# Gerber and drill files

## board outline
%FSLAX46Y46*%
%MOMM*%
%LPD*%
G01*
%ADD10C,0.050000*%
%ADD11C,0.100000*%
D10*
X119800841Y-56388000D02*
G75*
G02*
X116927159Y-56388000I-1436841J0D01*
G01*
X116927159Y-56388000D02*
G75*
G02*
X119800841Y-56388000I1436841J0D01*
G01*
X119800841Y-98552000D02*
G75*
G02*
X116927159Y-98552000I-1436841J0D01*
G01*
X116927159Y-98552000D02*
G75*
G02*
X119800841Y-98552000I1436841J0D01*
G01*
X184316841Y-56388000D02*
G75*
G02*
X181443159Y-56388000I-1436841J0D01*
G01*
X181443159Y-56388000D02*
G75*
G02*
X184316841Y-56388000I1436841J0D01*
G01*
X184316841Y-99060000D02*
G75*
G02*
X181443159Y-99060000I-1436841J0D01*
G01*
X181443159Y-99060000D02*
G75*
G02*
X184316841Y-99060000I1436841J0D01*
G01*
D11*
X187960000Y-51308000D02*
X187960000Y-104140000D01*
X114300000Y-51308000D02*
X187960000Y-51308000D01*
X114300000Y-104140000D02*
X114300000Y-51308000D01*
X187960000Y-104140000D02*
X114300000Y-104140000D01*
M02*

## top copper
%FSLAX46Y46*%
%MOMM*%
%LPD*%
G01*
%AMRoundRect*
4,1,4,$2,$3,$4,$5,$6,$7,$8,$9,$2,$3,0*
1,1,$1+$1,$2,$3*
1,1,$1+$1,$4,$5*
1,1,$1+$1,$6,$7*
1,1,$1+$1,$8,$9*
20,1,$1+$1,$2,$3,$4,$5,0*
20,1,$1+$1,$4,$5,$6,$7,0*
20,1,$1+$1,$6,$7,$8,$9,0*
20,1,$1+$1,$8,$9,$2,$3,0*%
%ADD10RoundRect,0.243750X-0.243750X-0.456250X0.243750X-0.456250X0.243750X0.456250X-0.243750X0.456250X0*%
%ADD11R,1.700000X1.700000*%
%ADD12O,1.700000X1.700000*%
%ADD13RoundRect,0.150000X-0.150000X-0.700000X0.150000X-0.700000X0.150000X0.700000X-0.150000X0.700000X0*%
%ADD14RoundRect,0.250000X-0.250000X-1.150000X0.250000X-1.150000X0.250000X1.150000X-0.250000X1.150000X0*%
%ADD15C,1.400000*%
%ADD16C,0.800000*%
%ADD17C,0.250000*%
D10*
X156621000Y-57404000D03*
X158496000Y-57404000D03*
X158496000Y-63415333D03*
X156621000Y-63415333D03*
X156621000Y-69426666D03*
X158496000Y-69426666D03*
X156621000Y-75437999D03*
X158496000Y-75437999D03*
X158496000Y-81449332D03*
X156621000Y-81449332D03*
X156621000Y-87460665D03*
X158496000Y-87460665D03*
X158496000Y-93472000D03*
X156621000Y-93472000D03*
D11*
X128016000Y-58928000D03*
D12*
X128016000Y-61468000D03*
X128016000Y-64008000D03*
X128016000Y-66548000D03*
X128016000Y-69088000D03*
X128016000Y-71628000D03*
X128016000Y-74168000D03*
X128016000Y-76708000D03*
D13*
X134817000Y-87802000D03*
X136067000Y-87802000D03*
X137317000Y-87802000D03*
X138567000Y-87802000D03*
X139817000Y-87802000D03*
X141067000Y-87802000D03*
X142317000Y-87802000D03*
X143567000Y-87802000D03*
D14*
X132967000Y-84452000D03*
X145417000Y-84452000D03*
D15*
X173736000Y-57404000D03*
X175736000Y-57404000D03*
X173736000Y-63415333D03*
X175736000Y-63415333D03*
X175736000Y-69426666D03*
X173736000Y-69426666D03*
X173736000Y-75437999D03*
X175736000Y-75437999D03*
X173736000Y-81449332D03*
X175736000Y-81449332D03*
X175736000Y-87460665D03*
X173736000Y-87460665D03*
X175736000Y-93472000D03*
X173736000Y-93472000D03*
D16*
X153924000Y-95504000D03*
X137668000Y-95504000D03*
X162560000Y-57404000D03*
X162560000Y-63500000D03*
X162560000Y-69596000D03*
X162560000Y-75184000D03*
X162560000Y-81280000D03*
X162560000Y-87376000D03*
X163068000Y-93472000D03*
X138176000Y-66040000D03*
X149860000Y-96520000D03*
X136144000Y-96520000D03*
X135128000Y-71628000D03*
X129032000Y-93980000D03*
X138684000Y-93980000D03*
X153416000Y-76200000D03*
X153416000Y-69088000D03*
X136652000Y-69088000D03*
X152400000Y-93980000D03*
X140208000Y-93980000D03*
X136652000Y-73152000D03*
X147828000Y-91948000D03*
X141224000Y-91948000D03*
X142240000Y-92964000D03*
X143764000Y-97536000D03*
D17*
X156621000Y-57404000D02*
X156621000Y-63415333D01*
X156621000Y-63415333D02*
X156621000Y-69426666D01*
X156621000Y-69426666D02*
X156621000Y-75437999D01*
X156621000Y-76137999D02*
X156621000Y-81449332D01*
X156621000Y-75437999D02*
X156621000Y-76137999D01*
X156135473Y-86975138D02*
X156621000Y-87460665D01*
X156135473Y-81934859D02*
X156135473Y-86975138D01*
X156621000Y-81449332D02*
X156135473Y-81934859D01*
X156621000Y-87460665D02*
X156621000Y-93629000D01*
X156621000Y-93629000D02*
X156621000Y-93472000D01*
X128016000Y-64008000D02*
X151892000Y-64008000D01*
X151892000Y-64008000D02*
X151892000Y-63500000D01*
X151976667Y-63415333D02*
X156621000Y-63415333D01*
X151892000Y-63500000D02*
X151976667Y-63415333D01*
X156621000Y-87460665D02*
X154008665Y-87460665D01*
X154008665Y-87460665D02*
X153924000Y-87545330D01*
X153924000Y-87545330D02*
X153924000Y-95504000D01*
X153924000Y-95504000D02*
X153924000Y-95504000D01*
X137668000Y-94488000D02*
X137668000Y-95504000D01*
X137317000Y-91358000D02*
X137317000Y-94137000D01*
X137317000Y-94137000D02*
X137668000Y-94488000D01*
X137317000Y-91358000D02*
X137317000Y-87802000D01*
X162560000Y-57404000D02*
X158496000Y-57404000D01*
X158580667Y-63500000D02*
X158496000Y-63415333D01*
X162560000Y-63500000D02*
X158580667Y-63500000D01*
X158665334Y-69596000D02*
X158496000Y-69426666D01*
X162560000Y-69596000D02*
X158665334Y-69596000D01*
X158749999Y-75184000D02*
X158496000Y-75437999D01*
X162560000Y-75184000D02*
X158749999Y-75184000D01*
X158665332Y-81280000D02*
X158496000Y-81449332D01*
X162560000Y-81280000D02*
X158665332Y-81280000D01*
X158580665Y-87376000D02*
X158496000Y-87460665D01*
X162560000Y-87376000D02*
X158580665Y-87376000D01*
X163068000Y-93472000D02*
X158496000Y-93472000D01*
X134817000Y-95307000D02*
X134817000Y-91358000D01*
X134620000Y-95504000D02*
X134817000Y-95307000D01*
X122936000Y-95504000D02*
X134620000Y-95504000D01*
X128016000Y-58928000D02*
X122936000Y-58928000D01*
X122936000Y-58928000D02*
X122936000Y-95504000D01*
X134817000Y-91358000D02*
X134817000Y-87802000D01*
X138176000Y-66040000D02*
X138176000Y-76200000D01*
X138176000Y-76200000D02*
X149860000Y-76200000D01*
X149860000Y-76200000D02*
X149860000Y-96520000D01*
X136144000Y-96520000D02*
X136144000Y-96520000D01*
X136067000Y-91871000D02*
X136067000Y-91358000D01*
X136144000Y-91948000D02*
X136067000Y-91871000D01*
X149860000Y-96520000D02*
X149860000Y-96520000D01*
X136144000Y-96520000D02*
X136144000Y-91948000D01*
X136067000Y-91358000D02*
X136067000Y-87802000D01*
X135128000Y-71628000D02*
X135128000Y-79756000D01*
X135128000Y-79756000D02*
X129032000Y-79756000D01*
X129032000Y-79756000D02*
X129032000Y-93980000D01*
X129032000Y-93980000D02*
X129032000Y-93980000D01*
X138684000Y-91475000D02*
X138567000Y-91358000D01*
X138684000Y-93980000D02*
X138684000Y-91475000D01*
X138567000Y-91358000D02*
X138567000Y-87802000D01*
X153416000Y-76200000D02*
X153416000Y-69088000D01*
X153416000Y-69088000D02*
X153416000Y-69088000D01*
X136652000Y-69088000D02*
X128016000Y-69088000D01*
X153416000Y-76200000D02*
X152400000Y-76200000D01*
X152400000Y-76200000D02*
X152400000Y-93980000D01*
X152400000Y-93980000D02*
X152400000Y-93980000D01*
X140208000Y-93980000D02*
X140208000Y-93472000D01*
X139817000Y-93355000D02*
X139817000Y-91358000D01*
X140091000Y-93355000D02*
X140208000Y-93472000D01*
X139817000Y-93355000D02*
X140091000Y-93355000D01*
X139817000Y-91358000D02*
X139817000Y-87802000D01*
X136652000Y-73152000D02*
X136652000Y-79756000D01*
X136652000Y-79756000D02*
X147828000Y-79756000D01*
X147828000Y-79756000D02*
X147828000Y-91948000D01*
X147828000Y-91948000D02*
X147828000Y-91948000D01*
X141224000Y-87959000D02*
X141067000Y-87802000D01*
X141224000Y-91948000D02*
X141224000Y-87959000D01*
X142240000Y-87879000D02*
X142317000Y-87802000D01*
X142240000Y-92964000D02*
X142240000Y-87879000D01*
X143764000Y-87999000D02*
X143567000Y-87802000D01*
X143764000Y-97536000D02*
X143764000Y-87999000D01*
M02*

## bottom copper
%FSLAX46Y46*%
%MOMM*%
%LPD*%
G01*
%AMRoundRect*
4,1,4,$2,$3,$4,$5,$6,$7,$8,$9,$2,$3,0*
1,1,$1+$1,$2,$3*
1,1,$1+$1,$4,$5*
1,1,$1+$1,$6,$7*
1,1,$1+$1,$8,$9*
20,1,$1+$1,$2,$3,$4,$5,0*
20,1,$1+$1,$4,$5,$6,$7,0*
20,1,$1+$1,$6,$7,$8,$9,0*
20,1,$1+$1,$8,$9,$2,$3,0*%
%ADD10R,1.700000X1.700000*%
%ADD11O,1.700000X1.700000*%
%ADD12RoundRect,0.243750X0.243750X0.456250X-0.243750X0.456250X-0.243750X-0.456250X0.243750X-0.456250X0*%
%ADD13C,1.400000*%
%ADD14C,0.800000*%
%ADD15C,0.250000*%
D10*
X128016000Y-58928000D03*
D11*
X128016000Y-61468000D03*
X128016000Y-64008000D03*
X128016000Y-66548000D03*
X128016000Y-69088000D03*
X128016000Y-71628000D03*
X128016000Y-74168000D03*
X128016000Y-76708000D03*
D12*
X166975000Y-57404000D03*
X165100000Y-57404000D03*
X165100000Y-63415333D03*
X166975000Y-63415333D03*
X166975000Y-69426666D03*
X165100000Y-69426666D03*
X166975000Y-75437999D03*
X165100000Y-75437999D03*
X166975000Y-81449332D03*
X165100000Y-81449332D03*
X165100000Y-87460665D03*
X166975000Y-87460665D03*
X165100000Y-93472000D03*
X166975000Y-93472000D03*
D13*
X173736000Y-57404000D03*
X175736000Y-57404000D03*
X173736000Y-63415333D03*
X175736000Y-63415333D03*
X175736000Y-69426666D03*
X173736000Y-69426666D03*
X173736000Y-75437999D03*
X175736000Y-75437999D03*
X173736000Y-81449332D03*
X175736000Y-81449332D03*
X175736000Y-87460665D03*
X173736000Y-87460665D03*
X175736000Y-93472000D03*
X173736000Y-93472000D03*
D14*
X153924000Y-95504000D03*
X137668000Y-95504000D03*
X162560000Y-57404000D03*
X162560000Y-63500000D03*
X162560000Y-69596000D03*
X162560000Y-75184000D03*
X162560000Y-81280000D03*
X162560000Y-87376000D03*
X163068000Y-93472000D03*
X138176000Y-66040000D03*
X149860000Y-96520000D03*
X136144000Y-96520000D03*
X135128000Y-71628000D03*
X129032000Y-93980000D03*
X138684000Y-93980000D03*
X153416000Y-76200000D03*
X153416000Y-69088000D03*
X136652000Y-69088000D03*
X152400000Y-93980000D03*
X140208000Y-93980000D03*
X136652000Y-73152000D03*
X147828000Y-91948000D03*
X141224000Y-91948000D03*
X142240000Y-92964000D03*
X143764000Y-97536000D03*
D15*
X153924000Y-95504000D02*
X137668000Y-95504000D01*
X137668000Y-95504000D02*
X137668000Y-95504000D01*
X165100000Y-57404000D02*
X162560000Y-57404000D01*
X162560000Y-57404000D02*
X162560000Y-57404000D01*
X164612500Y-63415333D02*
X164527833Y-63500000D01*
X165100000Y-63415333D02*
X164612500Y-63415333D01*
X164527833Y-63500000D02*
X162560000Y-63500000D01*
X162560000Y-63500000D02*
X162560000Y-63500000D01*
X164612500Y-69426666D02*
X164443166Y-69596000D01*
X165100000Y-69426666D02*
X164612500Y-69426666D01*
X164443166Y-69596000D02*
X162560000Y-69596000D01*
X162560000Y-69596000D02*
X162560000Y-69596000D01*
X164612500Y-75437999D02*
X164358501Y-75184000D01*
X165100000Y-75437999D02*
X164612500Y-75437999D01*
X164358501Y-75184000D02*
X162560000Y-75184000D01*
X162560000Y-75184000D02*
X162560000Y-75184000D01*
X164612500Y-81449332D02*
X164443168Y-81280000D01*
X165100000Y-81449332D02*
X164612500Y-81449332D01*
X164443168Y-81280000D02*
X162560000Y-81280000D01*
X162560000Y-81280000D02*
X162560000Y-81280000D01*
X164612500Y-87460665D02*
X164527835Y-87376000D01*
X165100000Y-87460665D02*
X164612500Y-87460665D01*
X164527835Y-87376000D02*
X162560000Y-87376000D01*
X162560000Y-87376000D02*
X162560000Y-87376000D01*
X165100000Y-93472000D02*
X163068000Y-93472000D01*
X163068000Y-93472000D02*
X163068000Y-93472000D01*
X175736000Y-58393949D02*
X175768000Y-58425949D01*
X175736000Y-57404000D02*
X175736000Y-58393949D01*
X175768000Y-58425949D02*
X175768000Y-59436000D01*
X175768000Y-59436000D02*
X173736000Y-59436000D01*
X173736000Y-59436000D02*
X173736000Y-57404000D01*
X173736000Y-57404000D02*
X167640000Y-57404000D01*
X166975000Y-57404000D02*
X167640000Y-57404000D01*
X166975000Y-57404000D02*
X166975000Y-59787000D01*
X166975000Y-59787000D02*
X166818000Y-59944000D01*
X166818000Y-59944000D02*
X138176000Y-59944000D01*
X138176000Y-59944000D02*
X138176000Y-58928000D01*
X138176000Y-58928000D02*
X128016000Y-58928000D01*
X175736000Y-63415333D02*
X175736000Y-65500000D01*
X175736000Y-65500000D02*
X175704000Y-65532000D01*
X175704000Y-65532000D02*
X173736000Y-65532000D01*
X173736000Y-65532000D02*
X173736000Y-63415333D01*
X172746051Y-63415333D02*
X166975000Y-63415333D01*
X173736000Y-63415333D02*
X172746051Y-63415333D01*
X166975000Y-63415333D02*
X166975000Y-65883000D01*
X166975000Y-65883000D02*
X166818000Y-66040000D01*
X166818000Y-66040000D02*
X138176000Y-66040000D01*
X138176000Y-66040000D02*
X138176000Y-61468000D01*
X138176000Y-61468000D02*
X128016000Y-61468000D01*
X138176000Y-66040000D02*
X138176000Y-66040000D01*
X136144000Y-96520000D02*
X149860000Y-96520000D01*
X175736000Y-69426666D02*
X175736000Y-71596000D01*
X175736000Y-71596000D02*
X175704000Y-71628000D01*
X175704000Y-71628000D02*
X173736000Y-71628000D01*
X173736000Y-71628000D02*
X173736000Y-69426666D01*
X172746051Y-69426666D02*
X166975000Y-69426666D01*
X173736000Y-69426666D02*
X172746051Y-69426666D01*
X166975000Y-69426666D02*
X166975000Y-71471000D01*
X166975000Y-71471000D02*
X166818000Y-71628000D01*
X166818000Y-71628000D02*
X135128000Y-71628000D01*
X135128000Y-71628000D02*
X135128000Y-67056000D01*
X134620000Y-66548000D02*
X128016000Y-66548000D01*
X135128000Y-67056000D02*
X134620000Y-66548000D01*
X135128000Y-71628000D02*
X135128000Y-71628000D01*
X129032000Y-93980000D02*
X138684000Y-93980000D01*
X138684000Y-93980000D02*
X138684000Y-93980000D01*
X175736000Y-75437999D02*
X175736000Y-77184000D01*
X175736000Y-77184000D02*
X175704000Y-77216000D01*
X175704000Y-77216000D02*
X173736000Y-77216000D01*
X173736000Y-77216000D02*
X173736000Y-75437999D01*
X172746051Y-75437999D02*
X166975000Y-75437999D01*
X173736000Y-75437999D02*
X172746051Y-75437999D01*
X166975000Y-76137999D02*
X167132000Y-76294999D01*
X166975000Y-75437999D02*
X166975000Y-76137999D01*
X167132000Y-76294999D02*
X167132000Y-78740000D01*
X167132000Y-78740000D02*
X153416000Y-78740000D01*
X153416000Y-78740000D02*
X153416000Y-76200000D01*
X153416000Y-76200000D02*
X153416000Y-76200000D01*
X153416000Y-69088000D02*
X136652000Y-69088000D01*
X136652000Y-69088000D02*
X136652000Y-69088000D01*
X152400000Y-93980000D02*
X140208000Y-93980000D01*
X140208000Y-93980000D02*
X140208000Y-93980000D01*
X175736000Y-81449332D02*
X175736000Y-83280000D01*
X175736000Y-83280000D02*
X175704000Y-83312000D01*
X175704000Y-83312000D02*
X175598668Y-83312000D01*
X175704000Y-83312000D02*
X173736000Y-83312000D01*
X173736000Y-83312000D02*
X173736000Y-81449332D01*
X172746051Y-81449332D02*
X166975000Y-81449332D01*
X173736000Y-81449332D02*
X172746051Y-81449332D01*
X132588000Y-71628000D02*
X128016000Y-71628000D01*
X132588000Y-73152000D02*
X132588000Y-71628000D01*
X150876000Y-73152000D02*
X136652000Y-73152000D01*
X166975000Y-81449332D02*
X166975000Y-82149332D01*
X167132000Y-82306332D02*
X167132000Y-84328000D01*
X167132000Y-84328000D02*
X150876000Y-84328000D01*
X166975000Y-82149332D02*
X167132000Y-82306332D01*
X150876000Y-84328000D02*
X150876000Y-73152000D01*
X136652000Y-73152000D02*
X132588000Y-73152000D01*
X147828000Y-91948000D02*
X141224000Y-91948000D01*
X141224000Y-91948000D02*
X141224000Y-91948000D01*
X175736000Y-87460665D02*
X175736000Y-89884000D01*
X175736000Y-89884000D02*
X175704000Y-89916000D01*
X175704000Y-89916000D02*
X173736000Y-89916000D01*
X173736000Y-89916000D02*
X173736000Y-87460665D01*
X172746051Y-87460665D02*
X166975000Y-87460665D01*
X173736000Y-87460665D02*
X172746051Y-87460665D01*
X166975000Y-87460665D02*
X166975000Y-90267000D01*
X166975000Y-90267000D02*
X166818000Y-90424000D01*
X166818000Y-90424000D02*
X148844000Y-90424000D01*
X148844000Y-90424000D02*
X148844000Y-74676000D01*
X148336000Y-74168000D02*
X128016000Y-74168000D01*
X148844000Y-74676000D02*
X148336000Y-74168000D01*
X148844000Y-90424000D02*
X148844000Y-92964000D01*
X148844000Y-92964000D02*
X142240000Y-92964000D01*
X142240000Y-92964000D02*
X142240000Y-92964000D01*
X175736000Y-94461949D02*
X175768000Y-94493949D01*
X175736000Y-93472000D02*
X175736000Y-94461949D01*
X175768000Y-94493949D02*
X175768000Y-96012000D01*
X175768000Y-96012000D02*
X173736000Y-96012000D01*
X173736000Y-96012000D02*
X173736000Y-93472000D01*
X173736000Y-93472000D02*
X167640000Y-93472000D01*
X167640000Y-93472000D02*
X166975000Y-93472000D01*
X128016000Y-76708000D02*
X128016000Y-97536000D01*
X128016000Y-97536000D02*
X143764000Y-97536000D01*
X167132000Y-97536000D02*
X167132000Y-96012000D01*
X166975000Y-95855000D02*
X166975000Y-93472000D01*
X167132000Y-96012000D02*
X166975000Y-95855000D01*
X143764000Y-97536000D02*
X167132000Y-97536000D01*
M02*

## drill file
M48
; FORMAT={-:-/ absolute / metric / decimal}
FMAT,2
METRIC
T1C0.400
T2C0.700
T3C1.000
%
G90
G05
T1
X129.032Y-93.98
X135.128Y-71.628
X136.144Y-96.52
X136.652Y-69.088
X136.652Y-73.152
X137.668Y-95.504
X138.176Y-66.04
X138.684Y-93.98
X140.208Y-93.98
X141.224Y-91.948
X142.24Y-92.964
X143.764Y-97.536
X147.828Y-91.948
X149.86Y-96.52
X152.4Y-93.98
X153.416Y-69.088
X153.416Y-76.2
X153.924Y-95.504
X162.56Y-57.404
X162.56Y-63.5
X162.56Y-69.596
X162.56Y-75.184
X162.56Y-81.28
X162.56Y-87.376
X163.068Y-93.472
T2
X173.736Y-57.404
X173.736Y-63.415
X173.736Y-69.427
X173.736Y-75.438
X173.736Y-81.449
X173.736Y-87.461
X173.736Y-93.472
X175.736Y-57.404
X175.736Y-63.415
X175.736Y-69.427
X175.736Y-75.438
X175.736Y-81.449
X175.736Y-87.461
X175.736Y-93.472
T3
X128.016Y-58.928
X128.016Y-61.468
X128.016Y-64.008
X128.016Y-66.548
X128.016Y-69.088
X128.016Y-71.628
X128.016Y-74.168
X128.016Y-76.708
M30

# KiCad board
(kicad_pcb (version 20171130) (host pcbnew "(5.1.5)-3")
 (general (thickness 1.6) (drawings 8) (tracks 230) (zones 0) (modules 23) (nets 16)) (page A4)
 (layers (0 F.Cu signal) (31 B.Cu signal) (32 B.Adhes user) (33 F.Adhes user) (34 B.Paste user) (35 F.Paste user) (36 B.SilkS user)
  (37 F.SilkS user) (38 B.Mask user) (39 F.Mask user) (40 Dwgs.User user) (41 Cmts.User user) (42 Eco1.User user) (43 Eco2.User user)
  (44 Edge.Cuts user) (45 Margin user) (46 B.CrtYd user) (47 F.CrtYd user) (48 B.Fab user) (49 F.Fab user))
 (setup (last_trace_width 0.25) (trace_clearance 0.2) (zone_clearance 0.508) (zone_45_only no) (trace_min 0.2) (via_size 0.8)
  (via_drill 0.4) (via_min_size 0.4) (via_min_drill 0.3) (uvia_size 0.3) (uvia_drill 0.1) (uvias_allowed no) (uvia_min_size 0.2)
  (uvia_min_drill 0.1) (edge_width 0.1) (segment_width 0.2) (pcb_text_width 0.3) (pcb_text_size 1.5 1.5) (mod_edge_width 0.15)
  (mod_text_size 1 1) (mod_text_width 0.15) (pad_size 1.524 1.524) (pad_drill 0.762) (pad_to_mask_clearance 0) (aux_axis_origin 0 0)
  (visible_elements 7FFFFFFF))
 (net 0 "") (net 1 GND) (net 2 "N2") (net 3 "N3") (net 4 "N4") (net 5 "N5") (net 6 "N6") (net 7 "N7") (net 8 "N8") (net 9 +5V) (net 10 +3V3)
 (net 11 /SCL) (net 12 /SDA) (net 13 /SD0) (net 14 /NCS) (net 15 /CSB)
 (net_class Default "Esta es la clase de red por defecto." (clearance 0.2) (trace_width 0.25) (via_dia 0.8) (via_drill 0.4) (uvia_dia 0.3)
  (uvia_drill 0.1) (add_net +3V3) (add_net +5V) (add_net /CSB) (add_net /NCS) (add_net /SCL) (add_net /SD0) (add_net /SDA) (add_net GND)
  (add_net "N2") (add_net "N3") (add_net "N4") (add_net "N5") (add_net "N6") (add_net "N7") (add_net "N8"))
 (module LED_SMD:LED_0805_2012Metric (layer F.Cu) (at 157.5585 57.404)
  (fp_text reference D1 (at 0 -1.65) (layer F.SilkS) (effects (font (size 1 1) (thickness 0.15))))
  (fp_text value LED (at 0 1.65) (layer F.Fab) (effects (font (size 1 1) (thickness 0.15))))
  (pad 1 smd roundrect (at -0.9375 0) (size 0.975 1.4) (layers F.Cu F.Paste F.Mask) (roundrect_rratio 0.25) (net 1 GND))
  (pad 2 smd roundrect (at 0.9375 0) (size 0.975 1.4) (layers F.Cu F.Paste F.Mask) (roundrect_rratio 0.25) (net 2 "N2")))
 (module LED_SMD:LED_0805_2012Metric (layer F.Cu) (at 157.5585 63.415333)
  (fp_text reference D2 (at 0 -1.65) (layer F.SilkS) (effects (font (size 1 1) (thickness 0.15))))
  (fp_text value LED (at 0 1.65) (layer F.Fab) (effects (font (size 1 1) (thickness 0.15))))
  (pad 2 smd roundrect (at 0.9375 0) (size 0.975 1.4) (layers F.Cu F.Paste F.Mask) (roundrect_rratio 0.25) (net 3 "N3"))
  (pad 1 smd roundrect (at -0.9375 0) (size 0.975 1.4) (layers F.Cu F.Paste F.Mask) (roundrect_rratio 0.25) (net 1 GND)))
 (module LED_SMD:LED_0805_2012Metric (layer F.Cu) (at 157.5585 69.426666)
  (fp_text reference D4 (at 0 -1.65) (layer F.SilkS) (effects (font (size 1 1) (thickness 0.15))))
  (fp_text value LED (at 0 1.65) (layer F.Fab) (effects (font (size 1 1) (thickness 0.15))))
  (pad 1 smd roundrect (at -0.9375 0) (size 0.975 1.4) (layers F.Cu F.Paste F.Mask) (roundrect_rratio 0.25) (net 1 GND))
  (pad 2 smd roundrect (at 0.9375 0) (size 0.975 1.4) (layers F.Cu F.Paste F.Mask) (roundrect_rratio 0.25) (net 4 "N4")))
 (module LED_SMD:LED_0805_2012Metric (layer F.Cu) (at 157.5585 75.437999)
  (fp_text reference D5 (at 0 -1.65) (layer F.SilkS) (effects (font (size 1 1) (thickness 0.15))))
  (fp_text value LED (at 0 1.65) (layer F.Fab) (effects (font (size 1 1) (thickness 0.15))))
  (pad 1 smd roundrect (at -0.9375 0) (size 0.975 1.4) (layers F.Cu F.Paste F.Mask) (roundrect_rratio 0.25) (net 1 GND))
  (pad 2 smd roundrect (at 0.9375 0) (size 0.975 1.4) (layers F.Cu F.Paste F.Mask) (roundrect_rratio 0.25) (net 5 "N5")))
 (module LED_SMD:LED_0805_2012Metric (layer F.Cu) (at 157.5585 81.449332)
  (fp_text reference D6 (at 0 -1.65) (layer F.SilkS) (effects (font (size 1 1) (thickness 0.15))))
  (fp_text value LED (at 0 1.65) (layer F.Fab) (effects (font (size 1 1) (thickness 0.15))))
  (pad 2 smd roundrect (at 0.9375 0) (size 0.975 1.4) (layers F.Cu F.Paste F.Mask) (roundrect_rratio 0.25) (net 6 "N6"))
  (pad 1 smd roundrect (at -0.9375 0) (size 0.975 1.4) (layers F.Cu F.Paste F.Mask) (roundrect_rratio 0.25) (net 1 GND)))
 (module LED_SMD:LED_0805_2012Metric (layer F.Cu) (at 157.5585 87.460665)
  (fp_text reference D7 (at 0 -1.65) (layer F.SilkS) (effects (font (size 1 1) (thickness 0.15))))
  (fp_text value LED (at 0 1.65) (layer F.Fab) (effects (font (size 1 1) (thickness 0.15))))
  (pad 1 smd roundrect (at -0.9375 0) (size 0.975 1.4) (layers F.Cu F.Paste F.Mask) (roundrect_rratio 0.25) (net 1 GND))
  (pad 2 smd roundrect (at 0.9375 0) (size 0.975 1.4) (layers F.Cu F.Paste F.Mask) (roundrect_rratio 0.25) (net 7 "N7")))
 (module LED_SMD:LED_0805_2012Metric (layer F.Cu) (at 157.5585 93.472)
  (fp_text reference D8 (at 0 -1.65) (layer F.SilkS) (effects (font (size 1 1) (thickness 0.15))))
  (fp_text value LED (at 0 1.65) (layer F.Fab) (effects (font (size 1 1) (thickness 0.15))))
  (pad 2 smd roundrect (at 0.9375 0) (size 0.975 1.4) (layers F.Cu F.Paste F.Mask) (roundrect_rratio 0.25) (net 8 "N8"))
  (pad 1 smd roundrect (at -0.9375 0) (size 0.975 1.4) (layers F.Cu F.Paste F.Mask) (roundrect_rratio 0.25) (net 1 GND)))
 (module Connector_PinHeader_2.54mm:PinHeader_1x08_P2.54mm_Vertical (layer F.Cu) (at 128.016 58.928)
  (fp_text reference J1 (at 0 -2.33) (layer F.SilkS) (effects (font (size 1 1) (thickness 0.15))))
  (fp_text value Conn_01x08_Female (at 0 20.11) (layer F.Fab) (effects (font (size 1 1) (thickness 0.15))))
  (pad 1 thru_hole rect (at 0 0) (size 1.7 1.7) (drill 1) (layers *.Cu *.Mask) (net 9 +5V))
  (pad 2 thru_hole oval (at 0 2.54) (size 1.7 1.7) (drill 1) (layers *.Cu *.Mask) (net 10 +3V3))
  (pad 3 thru_hole oval (at 0 5.08) (size 1.7 1.7) (drill 1) (layers *.Cu *.Mask) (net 1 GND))
  (pad 4 thru_hole oval (at 0 7.62) (size 1.7 1.7) (drill 1) (layers *.Cu *.Mask) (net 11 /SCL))
  (pad 5 thru_hole oval (at 0 10.16) (size 1.7 1.7) (drill 1) (layers *.Cu *.Mask) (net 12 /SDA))
  (pad 6 thru_hole oval (at 0 12.7) (size 1.7 1.7) (drill 1) (layers *.Cu *.Mask) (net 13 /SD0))
  (pad 7 thru_hole oval (at 0 15.24) (size 1.7 1.7) (drill 1) (layers *.Cu *.Mask) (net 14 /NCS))
  (pad 8 thru_hole oval (at 0 17.78) (size 1.7 1.7) (drill 1) (layers *.Cu *.Mask) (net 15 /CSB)))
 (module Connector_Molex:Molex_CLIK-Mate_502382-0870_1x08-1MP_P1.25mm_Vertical (layer F.Cu) (at 139.192 85.852)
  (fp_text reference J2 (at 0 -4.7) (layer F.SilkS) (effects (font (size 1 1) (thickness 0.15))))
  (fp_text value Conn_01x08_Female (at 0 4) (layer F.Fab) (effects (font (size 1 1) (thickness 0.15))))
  (pad 1 smd roundrect (at -4.375 1.95) (size 0.6 1.7) (layers F.Cu F.Paste F.Mask) (roundrect_rratio 0.25) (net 9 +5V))
  (pad 2 smd roundrect (at -3.125 1.95) (size 0.6 1.7) (layers F.Cu F.Paste F.Mask) (roundrect_rratio 0.25) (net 10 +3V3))
  (pad 3 smd roundrect (at -1.875 1.95) (size 0.6 1.7) (layers F.Cu F.Paste F.Mask) (roundrect_rratio 0.25) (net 1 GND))
  (pad 4 smd roundrect (at -0.625 1.95) (size 0.6 1.7) (layers F.Cu F.Paste F.Mask) (roundrect_rratio 0.25) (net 11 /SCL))
  (pad 5 smd roundrect (at 0.625 1.95) (size 0.6 1.7) (layers F.Cu F.Paste F.Mask) (roundrect_rratio 0.25) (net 12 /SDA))
  (pad 6 smd roundrect (at 1.875 1.95) (size 0.6 1.7) (layers F.Cu F.Paste F.Mask) (roundrect_rratio 0.25) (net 13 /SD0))
  (pad 7 smd roundrect (at 3.125 1.95) (size 0.6 1.7) (layers F.Cu F.Paste F.Mask) (roundrect_rratio 0.25) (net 14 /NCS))
  (pad 8 smd roundrect (at 4.375 1.95) (size 0.6 1.7) (layers F.Cu F.Paste F.Mask) (roundrect_rratio 0.25) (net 15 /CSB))
  (pad MP smd roundrect (at -6.225 -1.4) (size 1 2.8) (layers F.Cu F.Paste F.Mask) (roundrect_rratio 0.25))
  (pad MP smd roundrect (at 6.225 -1.4) (size 1 2.8) (layers F.Cu F.Paste F.Mask) (roundrect_rratio 0.25)))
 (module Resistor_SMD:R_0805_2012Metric (layer B.Cu) (at 166.0375 57.404 180)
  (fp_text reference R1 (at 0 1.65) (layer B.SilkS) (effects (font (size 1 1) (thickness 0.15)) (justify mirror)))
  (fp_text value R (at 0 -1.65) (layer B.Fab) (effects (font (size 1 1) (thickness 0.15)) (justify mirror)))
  (pad 1 smd roundrect (at -0.9375 0 180) (size 0.975 1.4) (layers B.Cu B.Paste B.Mask) (roundrect_rratio 0.25) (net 9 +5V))
  (pad 2 smd roundrect (at 0.9375 0 180) (size 0.975 1.4) (layers B.Cu B.Paste B.Mask) (roundrect_rratio 0.25) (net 2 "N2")))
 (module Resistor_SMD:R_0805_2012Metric (layer B.Cu) (at 166.0375 63.415333 180)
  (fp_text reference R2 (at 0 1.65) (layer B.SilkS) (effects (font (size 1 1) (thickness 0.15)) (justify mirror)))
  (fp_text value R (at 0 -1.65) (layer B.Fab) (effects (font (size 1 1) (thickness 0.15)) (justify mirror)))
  (pad 2 smd roundrect (at 0.9375 0 180) (size 0.975 1.4) (layers B.Cu B.Paste B.Mask) (roundrect_rratio 0.25) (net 3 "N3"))
  (pad 1 smd roundrect (at -0.9375 0 180) (size 0.975 1.4) (layers B.Cu B.Paste B.Mask) (roundrect_rratio 0.25) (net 10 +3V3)))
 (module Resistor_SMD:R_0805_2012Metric (layer B.Cu) (at 166.0375 69.426666 180)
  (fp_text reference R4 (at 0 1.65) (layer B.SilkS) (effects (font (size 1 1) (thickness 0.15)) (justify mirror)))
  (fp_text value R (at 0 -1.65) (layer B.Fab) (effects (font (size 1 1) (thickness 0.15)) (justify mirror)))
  (pad 1 smd roundrect (at -0.9375 0 180) (size 0.975 1.4) (layers B.Cu B.Paste B.Mask) (roundrect_rratio 0.25) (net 11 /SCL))
  (pad 2 smd roundrect (at 0.9375 0 180) (size 0.975 1.4) (layers B.Cu B.Paste B.Mask) (roundrect_rratio 0.25) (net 4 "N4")))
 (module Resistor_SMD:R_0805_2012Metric (layer B.Cu) (at 166.0375 75.437999 180)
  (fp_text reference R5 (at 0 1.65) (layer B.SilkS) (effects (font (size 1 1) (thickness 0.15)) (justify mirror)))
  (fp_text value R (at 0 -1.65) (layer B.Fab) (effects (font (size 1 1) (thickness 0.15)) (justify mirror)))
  (pad 1 smd roundrect (at -0.9375 0 180) (size 0.975 1.4) (layers B.Cu B.Paste B.Mask) (roundrect_rratio 0.25) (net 12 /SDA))
  (pad 2 smd roundrect (at 0.9375 0 180) (size 0.975 1.4) (layers B.Cu B.Paste B.Mask) (roundrect_rratio 0.25) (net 5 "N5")))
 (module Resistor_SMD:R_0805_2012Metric (layer B.Cu) (at 166.0375 81.449332 180)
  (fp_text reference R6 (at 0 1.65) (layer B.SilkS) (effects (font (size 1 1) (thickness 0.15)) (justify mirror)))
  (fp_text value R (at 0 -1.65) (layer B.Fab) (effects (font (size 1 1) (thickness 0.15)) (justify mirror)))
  (pad 1 smd roundrect (at -0.9375 0 180) (size 0.975 1.4) (layers B.Cu B.Paste B.Mask) (roundrect_rratio 0.25) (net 13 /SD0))
  (pad 2 smd roundrect (at 0.9375 0 180) (size 0.975 1.4) (layers B.Cu B.Paste B.Mask) (roundrect_rratio 0.25) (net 6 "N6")))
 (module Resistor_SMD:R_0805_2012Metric (layer B.Cu) (at 166.0375 87.460665 180)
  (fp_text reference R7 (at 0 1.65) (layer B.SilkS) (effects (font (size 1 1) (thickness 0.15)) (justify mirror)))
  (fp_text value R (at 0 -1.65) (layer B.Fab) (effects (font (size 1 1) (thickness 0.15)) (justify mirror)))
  (pad 2 smd roundrect (at 0.9375 0 180) (size 0.975 1.4) (layers B.Cu B.Paste B.Mask) (roundrect_rratio 0.25) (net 7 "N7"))
  (pad 1 smd roundrect (at -0.9375 0 180) (size 0.975 1.4) (layers B.Cu B.Paste B.Mask) (roundrect_rratio 0.25) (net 14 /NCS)))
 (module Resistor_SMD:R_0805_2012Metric (layer B.Cu) (at 166.0375 93.472 180)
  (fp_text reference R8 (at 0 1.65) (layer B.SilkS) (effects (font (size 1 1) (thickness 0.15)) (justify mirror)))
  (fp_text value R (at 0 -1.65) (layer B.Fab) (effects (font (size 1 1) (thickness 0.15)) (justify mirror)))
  (pad 2 smd roundrect (at 0.9375 0 180) (size 0.975 1.4) (layers B.Cu B.Paste B.Mask) (roundrect_rratio 0.25) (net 8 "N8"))
  (pad 1 smd roundrect (at -0.9375 0 180) (size 0.975 1.4) (layers B.Cu B.Paste B.Mask) (roundrect_rratio 0.25) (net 15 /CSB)))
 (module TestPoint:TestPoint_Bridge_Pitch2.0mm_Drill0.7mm (layer F.Cu) (at 173.736 57.404)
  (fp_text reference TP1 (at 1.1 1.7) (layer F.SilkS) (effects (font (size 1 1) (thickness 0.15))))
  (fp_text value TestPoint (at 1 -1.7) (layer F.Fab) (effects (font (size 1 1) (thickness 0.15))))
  (pad 1 thru_hole circle (at 0 0) (size 1.4 1.4) (drill 0.7) (layers *.Cu *.Mask) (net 9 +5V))
  (pad 1 thru_hole circle (at 2 0) (size 1.4 1.4) (drill 0.7) (layers *.Cu *.Mask) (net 9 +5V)))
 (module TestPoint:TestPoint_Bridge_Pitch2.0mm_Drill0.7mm (layer F.Cu) (at 173.736 63.415333)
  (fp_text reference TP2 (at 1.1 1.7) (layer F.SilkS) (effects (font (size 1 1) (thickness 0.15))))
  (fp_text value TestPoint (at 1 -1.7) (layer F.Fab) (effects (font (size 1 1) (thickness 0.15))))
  (pad 1 thru_hole circle (at 0 0) (size 1.4 1.4) (drill 0.7) (layers *.Cu *.Mask) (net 10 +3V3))
  (pad 1 thru_hole circle (at 2 0) (size 1.4 1.4) (drill 0.7) (layers *.Cu *.Mask) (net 10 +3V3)))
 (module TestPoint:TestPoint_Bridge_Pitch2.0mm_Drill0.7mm (layer F.Cu) (at 173.736 69.426666)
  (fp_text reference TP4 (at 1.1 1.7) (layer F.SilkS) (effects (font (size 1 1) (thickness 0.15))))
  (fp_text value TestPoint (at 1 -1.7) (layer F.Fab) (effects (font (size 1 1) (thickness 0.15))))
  (pad 1 thru_hole circle (at 2 0) (size 1.4 1.4) (drill 0.7) (layers *.Cu *.Mask) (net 11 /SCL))
  (pad 1 thru_hole circle (at 0 0) (size 1.4 1.4) (drill 0.7) (layers *.Cu *.Mask) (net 11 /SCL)))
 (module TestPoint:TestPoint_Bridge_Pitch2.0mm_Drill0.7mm (layer F.Cu) (at 173.736 75.437999)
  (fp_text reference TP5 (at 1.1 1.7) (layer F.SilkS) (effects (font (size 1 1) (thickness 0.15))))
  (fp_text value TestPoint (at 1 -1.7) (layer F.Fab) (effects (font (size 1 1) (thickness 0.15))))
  (pad 1 thru_hole circle (at 0 0) (size 1.4 1.4) (drill 0.7) (layers *.Cu *.Mask) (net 12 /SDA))
  (pad 1 thru_hole circle (at 2 0) (size 1.4 1.4) (drill 0.7) (layers *.Cu *.Mask) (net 12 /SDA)))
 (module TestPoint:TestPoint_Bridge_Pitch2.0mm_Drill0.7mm (layer F.Cu) (at 173.736 81.449332)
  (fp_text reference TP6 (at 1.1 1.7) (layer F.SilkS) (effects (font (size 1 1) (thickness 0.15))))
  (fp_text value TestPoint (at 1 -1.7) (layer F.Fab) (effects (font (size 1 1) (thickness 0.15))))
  (pad 1 thru_hole circle (at 0 0) (size 1.4 1.4) (drill 0.7) (layers *.Cu *.Mask) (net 13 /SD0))
  (pad 1 thru_hole circle (at 2 0) (size 1.4 1.4) (drill 0.7) (layers *.Cu *.Mask) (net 13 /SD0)))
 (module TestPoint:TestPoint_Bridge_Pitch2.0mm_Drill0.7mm (layer F.Cu) (at 173.736 87.460665)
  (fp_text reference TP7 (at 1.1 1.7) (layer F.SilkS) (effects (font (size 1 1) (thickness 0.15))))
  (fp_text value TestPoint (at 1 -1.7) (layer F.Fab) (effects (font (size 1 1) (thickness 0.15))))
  (pad 1 thru_hole circle (at 2 0) (size 1.4 1.4) (drill 0.7) (layers *.Cu *.Mask) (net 14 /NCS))
  (pad 1 thru_hole circle (at 0 0) (size 1.4 1.4) (drill 0.7) (layers *.Cu *.Mask) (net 14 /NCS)))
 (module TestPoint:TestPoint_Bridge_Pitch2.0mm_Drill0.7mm (layer F.Cu) (at 173.736 93.472)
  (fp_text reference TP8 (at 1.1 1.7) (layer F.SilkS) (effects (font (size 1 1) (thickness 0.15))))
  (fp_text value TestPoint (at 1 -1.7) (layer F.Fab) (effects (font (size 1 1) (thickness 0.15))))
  (pad 1 thru_hole circle (at 2 0) (size 1.4 1.4) (drill 0.7) (layers *.Cu *.Mask) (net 15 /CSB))
  (pad 1 thru_hole circle (at 0 0) (size 1.4 1.4) (drill 0.7) (layers *.Cu *.Mask) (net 15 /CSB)))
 (gr_circle (center 118.364 56.388) (end 119.38 57.404) (layer Edge.Cuts) (width 0.05))
 (gr_circle (center 118.364 98.552) (end 119.38 99.568) (layer Edge.Cuts) (width 0.05))
 (gr_circle (center 182.88 56.388) (end 183.896 57.404) (layer Edge.Cuts) (width 0.05))
 (gr_circle (center 182.88 99.06) (end 183.896 100.076) (layer Edge.Cuts) (width 0.05))
 (gr_line (start 187.96 51.308) (end 187.96 104.14) (layer Edge.Cuts) (width 0.1))
 (gr_line (start 114.3 51.308) (end 187.96 51.308) (layer Edge.Cuts) (width 0.1))
 (gr_line (start 114.3 104.14) (end 114.3 51.308) (layer Edge.Cuts) (width 0.1))
 (gr_line (start 187.96 104.14) (end 114.3 104.14) (layer Edge.Cuts) (width 0.1))
 (segment (start 156.621 57.404) (end 156.621 63.415333) (width 0.25) (layer F.Cu) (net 1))
 (segment (start 156.621 63.415333) (end 156.621 69.426666) (width 0.25) (layer F.Cu) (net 1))
 (segment (start 156.621 69.426666) (end 156.621 75.437999) (width 0.25) (layer F.Cu) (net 1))
 (segment (start 156.621 76.137999) (end 156.621 81.449332) (width 0.25) (layer F.Cu) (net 1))
 (segment (start 156.621 75.437999) (end 156.621 76.137999) (width 0.25) (layer F.Cu) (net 1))
 (segment (start 156.135473 86.975138) (end 156.621 87.460665) (width 0.25) (layer F.Cu) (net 1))
 (segment (start 156.135473 81.934859) (end 156.135473 86.975138) (width 0.25) (layer F.Cu) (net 1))
 (segment (start 156.621 81.449332) (end 156.135473 81.934859) (width 0.25) (layer F.Cu) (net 1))
 (segment (start 156.621 87.460665) (end 156.621 93.629) (width 0.25) (layer F.Cu) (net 1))
 (segment (start 156.621 93.629) (end 156.621 93.472) (width 0.25) (layer F.Cu) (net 1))
 (segment (start 128.016 64.008) (end 151.892 64.008) (width 0.25) (layer F.Cu) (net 1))
 (segment (start 151.892 64.008) (end 151.892 63.5) (width 0.25) (layer F.Cu) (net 1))
 (segment (start 151.976667 63.415333) (end 156.621 63.415333) (width 0.25) (layer F.Cu) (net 1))
 (segment (start 151.892 63.5) (end 151.976667 63.415333) (width 0.25) (layer F.Cu) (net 1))
 (segment (start 156.621 87.460665) (end 154.008665 87.460665) (width 0.25) (layer F.Cu) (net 1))
 (segment (start 154.008665 87.460665) (end 153.924 87.54533) (width 0.25) (layer F.Cu) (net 1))
 (segment (start 153.924 87.54533) (end 153.924 95.504) (width 0.25) (layer F.Cu) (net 1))
 (segment (start 153.924 95.504) (end 153.924 95.504) (width 0.25) (layer F.Cu) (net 1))
 (via (at 153.924 95.504) (size 0.8) (drill 0.4) (layers F.Cu B.Cu) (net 1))
 (segment (start 153.924 95.504) (end 137.668 95.504) (width 0.25) (layer B.Cu) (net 1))
 (segment (start 137.668 95.504) (end 137.668 95.504) (width 0.25) (layer B.Cu) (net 1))
 (via (at 137.668 95.504) (size 0.8) (drill 0.4) (layers F.Cu B.Cu) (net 1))
 (segment (start 137.668 94.488) (end 137.668 95.504) (width 0.25) (layer F.Cu) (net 1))
 (segment (start 137.317 91.358) (end 137.317 94.137) (width 0.25) (layer F.Cu) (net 1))
 (segment (start 137.317 94.137) (end 137.668 94.488) (width 0.25) (layer F.Cu) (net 1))
 (segment (start 137.317 91.358) (end 137.317 87.802) (width 0.25) (layer F.Cu) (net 1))
 (segment (start 165.1 57.404) (end 162.56 57.404) (width 0.25) (layer B.Cu) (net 2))
 (segment (start 162.56 57.404) (end 162.56 57.404) (width 0.25) (layer B.Cu) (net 2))
 (via (at 162.56 57.404) (size 0.8) (drill 0.4) (layers F.Cu B.Cu) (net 2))
 (segment (start 162.56 57.404) (end 158.496 57.404) (width 0.25) (layer F.Cu) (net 2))
 (segment (start 164.6125 63.415333) (end 164.527833 63.5) (width 0.25) (layer B.Cu) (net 3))
 (segment (start 165.1 63.415333) (end 164.6125 63.415333) (width 0.25) (layer B.Cu) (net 3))
 (segment (start 164.527833 63.5) (end 162.56 63.5) (width 0.25) (layer B.Cu) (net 3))
 (segment (start 162.56 63.5) (end 162.56 63.5) (width 0.25) (layer B.Cu) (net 3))
 (via (at 162.56 63.5) (size 0.8) (drill 0.4) (layers F.Cu B.Cu) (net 3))
 (segment (start 158.580667 63.5) (end 158.496 63.415333) (width 0.25) (layer F.Cu) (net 3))
 (segment (start 162.56 63.5) (end 158.580667 63.5) (width 0.25) (layer F.Cu) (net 3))
 (segment (start 164.6125 69.426666) (end 164.443166 69.596) (width 0.25) (layer B.Cu) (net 4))
 (segment (start 165.1 69.426666) (end 164.6125 69.426666) (width 0.25) (layer B.Cu) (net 4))
 (segment (start 164.443166 69.596) (end 162.56 69.596) (width 0.25) (layer B.Cu) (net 4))
 (segment (start 162.56 69.596) (end 162.56 69.596) (width 0.25) (layer B.Cu) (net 4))
 (via (at 162.56 69.596) (size 0.8) (drill 0.4) (layers F.Cu B.Cu) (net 4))
 (segment (start 158.665334 69.596) (end 158.496 69.426666) (width 0.25) (layer F.Cu) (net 4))
 (segment (start 162.56 69.596) (end 158.665334 69.596) (width 0.25) (layer F.Cu) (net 4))
 (segment (start 164.6125 75.437999) (end 164.358501 75.184) (width 0.25) (layer B.Cu) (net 5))
 (segment (start 165.1 75.437999) (end 164.6125 75.437999) (width 0.25) (layer B.Cu) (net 5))
 (segment (start 164.358501 75.184) (end 162.56 75.184) (width 0.25) (layer B.Cu) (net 5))
 (segment (start 162.56 75.184) (end 162.56 75.184) (width 0.25) (layer B.Cu) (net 5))
 (via (at 162.56 75.184) (size 0.8) (drill 0.4) (layers F.Cu B.Cu) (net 5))
 (segment (start 158.749999 75.184) (end 158.496 75.437999) (width 0.25) (layer F.Cu) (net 5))
 (segment (start 162.56 75.184) (end 158.749999 75.184) (width 0.25) (layer F.Cu) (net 5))
 (segment (start 164.6125 81.449332) (end 164.443168 81.28) (width 0.25) (layer B.Cu) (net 6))
 (segment (start 165.1 81.449332) (end 164.6125 81.449332) (width 0.25) (layer B.Cu) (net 6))
 (segment (start 164.443168 81.28) (end 162.56 81.28) (width 0.25) (layer B.Cu) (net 6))
 (segment (start 162.56 81.28) (end 162.56 81.28) (width 0.25) (layer B.Cu) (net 6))
 (via (at 162.56 81.28) (size 0.8) (drill 0.4) (layers F.Cu B.Cu) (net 6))
 (segment (start 158.665332 81.28) (end 158.496 81.449332) (width 0.25) (layer F.Cu) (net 6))
 (segment (start 162.56 81.28) (end 158.665332 81.28) (width 0.25) (layer F.Cu) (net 6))
 (segment (start 164.6125 87.460665) (end 164.527835 87.376) (width 0.25) (layer B.Cu) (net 7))
 (segment (start 165.1 87.460665) (end 164.6125 87.460665) (width 0.25) (layer B.Cu) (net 7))
 (segment (start 164.527835 87.376) (end 162.56 87.376) (width 0.25) (layer B.Cu) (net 7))
 (segment (start 162.56 87.376) (end 162.56 87.376) (width 0.25) (layer B.Cu) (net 7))
 (via (at 162.56 87.376) (size 0.8) (drill 0.4) (layers F.Cu B.Cu) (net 7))
 (segment (start 158.580665 87.376) (end 158.496 87.460665) (width 0.25) (layer F.Cu) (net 7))
 (segment (start 162.56 87.376) (end 158.580665 87.376) (width 0.25) (layer F.Cu) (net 7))
 (segment (start 165.1 93.472) (end 163.068 93.472) (width 0.25) (layer B.Cu) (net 8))
 (segment (start 163.068 93.472) (end 163.068 93.472) (width 0.25) (layer B.Cu) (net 8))
 (via (at 163.068 93.472) (size 0.8) (drill 0.4) (layers F.Cu B.Cu) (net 8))
 (segment (start 163.068 93.472) (end 158.496 93.472) (width 0.25) (layer F.Cu) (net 8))
 (segment (start 175.736 58.393949) (end 175.768 58.425949) (width 0.25) (layer B.Cu) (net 9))
 (segment (start 175.736 57.404) (end 175.736 58.393949) (width 0.25) (layer B.Cu) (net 9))
 (segment (start 175.768 58.425949) (end 175.768 59.436) (width 0.25) (layer B.Cu) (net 9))
 (segment (start 175.768 59.436) (end 173.736 59.436) (width 0.25) (layer B.Cu) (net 9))
 (segment (start 173.736 59.436) (end 173.736 57.404) (width 0.25) (layer B.Cu) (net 9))
 (segment (start 173.736 57.404) (end 167.64 57.404) (width 0.25) (layer B.Cu) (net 9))
 (segment (start 166.975 57.404) (end 167.64 57.404) (width 0.25) (layer B.Cu) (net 9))
 (segment (start 166.975 57.404) (end 166.975 59.787) (width 0.25) (layer B.Cu) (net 9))
 (segment (start 166.975 59.787) (end 166.818 59.944) (width 0.25) (layer B.Cu) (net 9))
 (segment (start 166.818 59.944) (end 138.176 59.944) (width 0.25) (layer B.Cu) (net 9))
 (segment (start 138.176 59.944) (end 138.176 58.928) (width 0.25) (layer B.Cu) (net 9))
 (segment (start 138.176 58.928) (end 128.016 58.928) (width 0.25) (layer B.Cu) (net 9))
 (segment (start 134.817 95.307) (end 134.817 91.358) (width 0.25) (layer F.Cu) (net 9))
 (segment (start 134.62 95.504) (end 134.817 95.307) (width 0.25) (layer F.Cu) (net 9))
 (segment (start 122.936 95.504) (end 134.62 95.504) (width 0.25) (layer F.Cu) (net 9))
 (segment (start 128.016 58.928) (end 122.936 58.928) (width 0.25) (layer F.Cu) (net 9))
 (segment (start 122.936 58.928) (end 122.936 95.504) (width 0.25) (layer F.Cu) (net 9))
 (segment (start 134.817 91.358) (end 134.817 87.802) (width 0.25) (layer F.Cu) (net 9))
 (segment (start 175.736 63.415333) (end 175.736 65.5) (width 0.25) (layer B.Cu) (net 10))
 (segment (start 175.736 65.5) (end 175.704 65.532) (width 0.25) (layer B.Cu) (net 10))
 (segment (start 175.704 65.532) (end 173.736 65.532) (width 0.25) (layer B.Cu) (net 10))
 (segment (start 173.736 65.532) (end 173.736 63.415333) (width 0.25) (layer B.Cu) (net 10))
 (segment (start 172.746051 63.415333) (end 166.975 63.415333) (width 0.25) (layer B.Cu) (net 10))
 (segment (start 173.736 63.415333) (end 172.746051 63.415333) (width 0.25) (layer B.Cu) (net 10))
 (segment (start 166.975 63.415333) (end 166.975 65.883) (width 0.25) (layer B.Cu) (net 10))
 (segment (start 166.975 65.883) (end 166.818 66.04) (width 0.25) (layer B.Cu) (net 10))
 (segment (start 166.818 66.04) (end 138.176 66.04) (width 0.25) (layer B.Cu) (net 10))
 (segment (start 138.176 66.04) (end 138.176 61.468) (width 0.25) (layer B.Cu) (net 10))
 (segment (start 138.176 61.468) (end 128.016 61.468) (width 0.25) (layer B.Cu) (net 10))
 (segment (start 138.176 66.04) (end 138.176 66.04) (width 0.25) (layer B.Cu) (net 10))
 (via (at 138.176 66.04) (size 0.8) (drill 0.4) (layers F.Cu B.Cu) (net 10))
 (segment (start 138.176 66.04) (end 138.176 76.2) (width 0.25) (layer F.Cu) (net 10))
 (segment (start 138.176 76.2) (end 149.86 76.2) (width 0.25) (layer F.Cu) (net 10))
 (segment (start 149.86 76.2) (end 149.86 96.52) (width 0.25) (layer F.Cu) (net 10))
 (segment (start 136.144 96.52) (end 136.144 96.52) (width 0.25) (layer F.Cu) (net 10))
 (segment (start 136.067 91.871) (end 136.067 91.358) (width 0.25) (layer F.Cu) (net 10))
 (segment (start 136.144 91.948) (end 136.067 91.871) (width 0.25) (layer F.Cu) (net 10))
 (segment (start 149.86 96.52) (end 149.86 96.52) (width 0.25) (layer F.Cu) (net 10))
 (via (at 149.86 96.52) (size 0.8) (drill 0.4) (layers F.Cu B.Cu) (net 10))
 (segment (start 136.144 96.52) (end 136.144 91.948) (width 0.25) (layer F.Cu) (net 10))
 (via (at 136.144 96.52) (size 0.8) (drill 0.4) (layers F.Cu B.Cu) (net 10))
 (segment (start 136.144 96.52) (end 149.86 96.52) (width 0.25) (layer B.Cu) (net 10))
 (segment (start 136.067 91.358) (end 136.067 87.802) (width 0.25) (layer F.Cu) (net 10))
 (segment (start 175.736 69.426666) (end 175.736 71.596) (width 0.25) (layer B.Cu) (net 11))
 (segment (start 175.736 71.596) (end 175.704 71.628) (width 0.25) (layer B.Cu) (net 11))
 (segment (start 175.704 71.628) (end 173.736 71.628) (width 0.25) (layer B.Cu) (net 11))
 (segment (start 173.736 71.628) (end 173.736 69.426666) (width 0.25) (layer B.Cu) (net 11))
 (segment (start 172.746051 69.426666) (end 166.975 69.426666) (width 0.25) (layer B.Cu) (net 11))
 (segment (start 173.736 69.426666) (end 172.746051 69.426666) (width 0.25) (layer B.Cu) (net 11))
 (segment (start 166.975 69.426666) (end 166.975 71.471) (width 0.25) (layer B.Cu) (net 11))
 (segment (start 166.975 71.471) (end 166.818 71.628) (width 0.25) (layer B.Cu) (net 11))
 (segment (start 166.818 71.628) (end 135.128 71.628) (width 0.25) (layer B.Cu) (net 11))
 (segment (start 135.128 71.628) (end 135.128 67.056) (width 0.25) (layer B.Cu) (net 11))
 (segment (start 134.62 66.548) (end 128.016 66.548) (width 0.25) (layer B.Cu) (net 11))
 (segment (start 135.128 67.056) (end 134.62 66.548) (width 0.25) (layer B.Cu) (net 11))
 (segment (start 135.128 71.628) (end 135.128 71.628) (width 0.25) (layer B.Cu) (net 11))
 (via (at 135.128 71.628) (size 0.8) (drill 0.4) (layers F.Cu B.Cu) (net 11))
 (segment (start 135.128 71.628) (end 135.128 79.756) (width 0.25) (layer F.Cu) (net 11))
 (segment (start 135.128 79.756) (end 129.032 79.756) (width 0.25) (layer F.Cu) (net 11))
 (segment (start 129.032 79.756) (end 129.032 93.98) (width 0.25) (layer F.Cu) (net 11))
 (segment (start 129.032 93.98) (end 129.032 93.98) (width 0.25) (layer F.Cu) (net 11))
 (via (at 129.032 93.98) (size 0.8) (drill 0.4) (layers F.Cu B.Cu) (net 11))
 (segment (start 129.032 93.98) (end 138.684 93.98) (width 0.25) (layer B.Cu) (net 11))
 (segment (start 138.684 93.98) (end 138.684 93.98) (width 0.25) (layer B.Cu) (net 11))
 (via (at 138.684 93.98) (size 0.8) (drill 0.4) (layers F.Cu B.Cu) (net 11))
 (segment (start 138.684 91.475) (end 138.567 91.358) (width 0.25) (layer F.Cu) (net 11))
 (segment (start 138.684 93.98) (end 138.684 91.475) (width 0.25) (layer F.Cu) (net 11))
 (segment (start 138.567 91.358) (end 138.567 87.802) (width 0.25) (layer F.Cu) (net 11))
 (segment (start 175.736 75.437999) (end 175.736 77.184) (width 0.25) (layer B.Cu) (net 12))
 (segment (start 175.736 77.184) (end 175.704 77.216) (width 0.25) (layer B.Cu) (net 12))
 (segment (start 175.704 77.216) (end 173.736 77.216) (width 0.25) (layer B.Cu) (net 12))
 (segment (start 173.736 77.216) (end 173.736 75.437999) (width 0.25) (layer B.Cu) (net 12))
 (segment (start 172.746051 75.437999) (end 166.975 75.437999) (width 0.25) (layer B.Cu) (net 12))
 (segment (start 173.736 75.437999) (end 172.746051 75.437999) (width 0.25) (layer B.Cu) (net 12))
 (segment (start 166.975 76.137999) (end 167.132 76.294999) (width 0.25) (layer B.Cu) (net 12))
 (segment (start 166.975 75.437999) (end 166.975 76.137999) (width 0.25) (layer B.Cu) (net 12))
 (segment (start 167.132 76.294999) (end 167.132 78.74) (width 0.25) (layer B.Cu) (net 12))
 (segment (start 167.132 78.74) (end 153.416 78.74) (width 0.25) (layer B.Cu) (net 12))
 (segment (start 153.416 78.74) (end 153.416 76.2) (width 0.25) (layer B.Cu) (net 12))
 (segment (start 153.416 76.2) (end 153.416 76.2) (width 0.25) (layer B.Cu) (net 12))
 (via (at 153.416 76.2) (size 0.8) (drill 0.4) (layers F.Cu B.Cu) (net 12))
 (segment (start 153.416 76.2) (end 153.416 69.088) (width 0.25) (layer F.Cu) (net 12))
 (segment (start 153.416 69.088) (end 153.416 69.088) (width 0.25) (layer F.Cu) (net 12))
 (via (at 153.416 69.088) (size 0.8) (drill 0.4) (layers F.Cu B.Cu) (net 12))
 (segment (start 153.416 69.088) (end 136.652 69.088) (width 0.25) (layer B.Cu) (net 12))
 (segment (start 136.652 69.088) (end 136.652 69.088) (width 0.25) (layer B.Cu) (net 12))
 (via (at 136.652 69.088) (size 0.8) (drill 0.4) (layers F.Cu B.Cu) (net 12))
 (segment (start 136.652 69.088) (end 128.016 69.088) (width 0.25) (layer F.Cu) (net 12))
 (segment (start 153.416 76.2) (end 152.4 76.2) (width 0.25) (layer F.Cu) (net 12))
 (segment (start 152.4 76.2) (end 152.4 93.98) (width 0.25) (layer F.Cu) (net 12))
 (segment (start 152.4 93.98) (end 152.4 93.98) (width 0.25) (layer F.Cu) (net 12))
 (via (at 152.4 93.98) (size 0.8) (drill 0.4) (layers F.Cu B.Cu) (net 12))
 (segment (start 152.4 93.98) (end 140.208 93.98) (width 0.25) (layer B.Cu) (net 12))
 (segment (start 140.208 93.98) (end 140.208 93.98) (width 0.25) (layer B.Cu) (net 12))
 (via (at 140.208 93.98) (size 0.8) (drill 0.4) (layers F.Cu B.Cu) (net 12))
 (segment (start 140.208 93.98) (end 140.208 93.472) (width 0.25) (layer F.Cu) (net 12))
 (segment (start 139.817 93.355) (end 139.817 91.358) (width 0.25) (layer F.Cu) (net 12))
 (segment (start 140.091 93.355) (end 140.208 93.472) (width 0.25) (layer F.Cu) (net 12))
 (segment (start 139.817 93.355) (end 140.091 93.355) (width 0.25) (layer F.Cu) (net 12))
 (segment (start 139.817 91.358) (end 139.817 87.802) (width 0.25) (layer F.Cu) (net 12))
 (segment (start 175.736 81.449332) (end 175.736 83.28) (width 0.25) (layer B.Cu) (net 13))
 (segment (start 175.736 83.28) (end 175.704 83.312) (width 0.25) (layer B.Cu) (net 13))
 (segment (start 175.704 83.312) (end 175.598668 83.312) (width 0.25) (layer B.Cu) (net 13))
 (segment (start 175.704 83.312) (end 173.736 83.312) (width 0.25) (layer B.Cu) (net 13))
 (segment (start 173.736 83.312) (end 173.736 81.449332) (width 0.25) (layer B.Cu) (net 13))
 (segment (start 172.746051 81.449332) (end 166.975 81.449332) (width 0.25) (layer B.Cu) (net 13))
 (segment (start 173.736 81.449332) (end 172.746051 81.449332) (width 0.25) (layer B.Cu) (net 13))
 (segment (start 132.588 71.628) (end 128.016 71.628) (width 0.25) (layer B.Cu) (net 13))
 (segment (start 132.588 73.152) (end 132.588 71.628) (width 0.25) (layer B.Cu) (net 13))
 (segment (start 150.876 73.152) (end 136.652 73.152) (width 0.25) (layer B.Cu) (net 13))
 (segment (start 166.975 81.449332) (end 166.975 82.149332) (width 0.25) (layer B.Cu) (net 13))
 (segment (start 167.132 82.306332) (end 167.132 84.328) (width 0.25) (layer B.Cu) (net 13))
 (segment (start 167.132 84.328) (end 150.876 84.328) (width 0.25) (layer B.Cu) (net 13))
 (segment (start 166.975 82.149332) (end 167.132 82.306332) (width 0.25) (layer B.Cu) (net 13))
 (segment (start 150.876 84.328) (end 150.876 73.152) (width 0.25) (layer B.Cu) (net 13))
 (segment (start 136.652 73.152) (end 132.588 73.152) (width 0.25) (layer B.Cu) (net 13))
 (via (at 136.652 73.152) (size 0.8) (drill 0.4) (layers F.Cu B.Cu) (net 13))
 (segment (start 136.652 73.152) (end 136.652 79.756) (width 0.25) (layer F.Cu) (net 13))
 (segment (start 136.652 79.756) (end 147.828 79.756) (width 0.25) (layer F.Cu) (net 13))
 (segment (start 147.828 79.756) (end 147.828 91.948) (width 0.25) (layer F.Cu) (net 13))
 (segment (start 147.828 91.948) (end 147.828 91.948) (width 0.25) (layer F.Cu) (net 13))
 (via (at 147.828 91.948) (size 0.8) (drill 0.4) (layers F.Cu B.Cu) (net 13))
 (segment (start 147.828 91.948) (end 141.224 91.948) (width 0.25) (layer B.Cu) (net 13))
 (segment (start 141.224 91.948) (end 141.224 91.948) (width 0.25) (layer B.Cu) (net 13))
 (via (at 141.224 91.948) (size 0.8) (drill 0.4) (layers F.Cu B.Cu) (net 13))
 (segment (start 141.224 87.959) (end 141.067 87.802) (width 0.25) (layer F.Cu) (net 13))
 (segment (start 141.224 91.948) (end 141.224 87.959) (width 0.25) (layer F.Cu) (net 13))
 (segment (start 175.736 87.460665) (end 175.736 89.884) (width 0.25) (layer B.Cu) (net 14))
 (segment (start 175.736 89.884) (end 175.704 89.916) (width 0.25) (layer B.Cu) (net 14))
 (segment (start 175.704 89.916) (end 173.736 89.916) (width 0.25) (layer B.Cu) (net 14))
 (segment (start 173.736 89.916) (end 173.736 87.460665) (width 0.25) (layer B.Cu) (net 14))
 (segment (start 172.746051 87.460665) (end 166.975 87.460665) (width 0.25) (layer B.Cu) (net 14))
 (segment (start 173.736 87.460665) (end 172.746051 87.460665) (width 0.25) (layer B.Cu) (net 14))
 (segment (start 166.975 87.460665) (end 166.975 90.267) (width 0.25) (layer B.Cu) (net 14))
 (segment (start 166.975 90.267) (end 166.818 90.424) (width 0.25) (layer B.Cu) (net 14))
 (segment (start 166.818 90.424) (end 148.844 90.424) (width 0.25) (layer B.Cu) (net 14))
 (segment (start 148.844 90.424) (end 148.844 74.676) (width 0.25) (layer B.Cu) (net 14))
 (segment (start 148.336 74.168) (end 128.016 74.168) (width 0.25) (layer B.Cu) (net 14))
 (segment (start 148.844 74.676) (end 148.336 74.168) (width 0.25) (layer B.Cu) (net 14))
 (segment (start 148.844 90.424) (end 148.844 92.964) (width 0.25) (layer B.Cu) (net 14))
 (segment (start 148.844 92.964) (end 142.24 92.964) (width 0.25) (layer B.Cu) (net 14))
 (segment (start 142.24 92.964) (end 142.24 92.964) (width 0.25) (layer B.Cu) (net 14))
 (via (at 142.24 92.964) (size 0.8) (drill 0.4) (layers F.Cu B.Cu) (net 14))
 (segment (start 142.24 87.879) (end 142.317 87.802) (width 0.25) (layer F.Cu) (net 14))
 (segment (start 142.24 92.964) (end 142.24 87.879) (width 0.25) (layer F.Cu) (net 14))
 (segment (start 175.736 94.461949) (end 175.768 94.493949) (width 0.25) (layer B.Cu) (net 15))
 (segment (start 175.736 93.472) (end 175.736 94.461949) (width 0.25) (layer B.Cu) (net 15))
 (segment (start 175.768 94.493949) (end 175.768 96.012) (width 0.25) (layer B.Cu) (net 15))
 (segment (start 175.768 96.012) (end 173.736 96.012) (width 0.25) (layer B.Cu) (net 15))
 (segment (start 173.736 96.012) (end 173.736 93.472) (width 0.25) (layer B.Cu) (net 15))
 (segment (start 173.736 93.472) (end 167.64 93.472) (width 0.25) (layer B.Cu) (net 15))
 (segment (start 167.64 93.472) (end 166.975 93.472) (width 0.25) (layer B.Cu) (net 15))
 (segment (start 128.016 76.708) (end 128.016 97.536) (width 0.25) (layer B.Cu) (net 15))
 (segment (start 128.016 97.536) (end 143.764 97.536) (width 0.25) (layer B.Cu) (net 15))
 (segment (start 167.132 97.536) (end 167.132 96.012) (width 0.25) (layer B.Cu) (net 15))
 (segment (start 166.975 95.855) (end 166.975 93.472) (width 0.25) (layer B.Cu) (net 15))
 (segment (start 167.132 96.012) (end 166.975 95.855) (width 0.25) (layer B.Cu) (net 15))
 (segment (start 143.764 97.536) (end 167.132 97.536) (width 0.25) (layer B.Cu) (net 15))
 (via (at 143.764 97.536) (size 0.8) (drill 0.4) (layers F.Cu B.Cu) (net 15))
 (segment (start 143.764 87.999) (end 143.567 87.802) (width 0.25) (layer F.Cu) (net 15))
 (segment (start 143.764 97.536) (end 143.764 87.999) (width 0.25) (layer F.Cu) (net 15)))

